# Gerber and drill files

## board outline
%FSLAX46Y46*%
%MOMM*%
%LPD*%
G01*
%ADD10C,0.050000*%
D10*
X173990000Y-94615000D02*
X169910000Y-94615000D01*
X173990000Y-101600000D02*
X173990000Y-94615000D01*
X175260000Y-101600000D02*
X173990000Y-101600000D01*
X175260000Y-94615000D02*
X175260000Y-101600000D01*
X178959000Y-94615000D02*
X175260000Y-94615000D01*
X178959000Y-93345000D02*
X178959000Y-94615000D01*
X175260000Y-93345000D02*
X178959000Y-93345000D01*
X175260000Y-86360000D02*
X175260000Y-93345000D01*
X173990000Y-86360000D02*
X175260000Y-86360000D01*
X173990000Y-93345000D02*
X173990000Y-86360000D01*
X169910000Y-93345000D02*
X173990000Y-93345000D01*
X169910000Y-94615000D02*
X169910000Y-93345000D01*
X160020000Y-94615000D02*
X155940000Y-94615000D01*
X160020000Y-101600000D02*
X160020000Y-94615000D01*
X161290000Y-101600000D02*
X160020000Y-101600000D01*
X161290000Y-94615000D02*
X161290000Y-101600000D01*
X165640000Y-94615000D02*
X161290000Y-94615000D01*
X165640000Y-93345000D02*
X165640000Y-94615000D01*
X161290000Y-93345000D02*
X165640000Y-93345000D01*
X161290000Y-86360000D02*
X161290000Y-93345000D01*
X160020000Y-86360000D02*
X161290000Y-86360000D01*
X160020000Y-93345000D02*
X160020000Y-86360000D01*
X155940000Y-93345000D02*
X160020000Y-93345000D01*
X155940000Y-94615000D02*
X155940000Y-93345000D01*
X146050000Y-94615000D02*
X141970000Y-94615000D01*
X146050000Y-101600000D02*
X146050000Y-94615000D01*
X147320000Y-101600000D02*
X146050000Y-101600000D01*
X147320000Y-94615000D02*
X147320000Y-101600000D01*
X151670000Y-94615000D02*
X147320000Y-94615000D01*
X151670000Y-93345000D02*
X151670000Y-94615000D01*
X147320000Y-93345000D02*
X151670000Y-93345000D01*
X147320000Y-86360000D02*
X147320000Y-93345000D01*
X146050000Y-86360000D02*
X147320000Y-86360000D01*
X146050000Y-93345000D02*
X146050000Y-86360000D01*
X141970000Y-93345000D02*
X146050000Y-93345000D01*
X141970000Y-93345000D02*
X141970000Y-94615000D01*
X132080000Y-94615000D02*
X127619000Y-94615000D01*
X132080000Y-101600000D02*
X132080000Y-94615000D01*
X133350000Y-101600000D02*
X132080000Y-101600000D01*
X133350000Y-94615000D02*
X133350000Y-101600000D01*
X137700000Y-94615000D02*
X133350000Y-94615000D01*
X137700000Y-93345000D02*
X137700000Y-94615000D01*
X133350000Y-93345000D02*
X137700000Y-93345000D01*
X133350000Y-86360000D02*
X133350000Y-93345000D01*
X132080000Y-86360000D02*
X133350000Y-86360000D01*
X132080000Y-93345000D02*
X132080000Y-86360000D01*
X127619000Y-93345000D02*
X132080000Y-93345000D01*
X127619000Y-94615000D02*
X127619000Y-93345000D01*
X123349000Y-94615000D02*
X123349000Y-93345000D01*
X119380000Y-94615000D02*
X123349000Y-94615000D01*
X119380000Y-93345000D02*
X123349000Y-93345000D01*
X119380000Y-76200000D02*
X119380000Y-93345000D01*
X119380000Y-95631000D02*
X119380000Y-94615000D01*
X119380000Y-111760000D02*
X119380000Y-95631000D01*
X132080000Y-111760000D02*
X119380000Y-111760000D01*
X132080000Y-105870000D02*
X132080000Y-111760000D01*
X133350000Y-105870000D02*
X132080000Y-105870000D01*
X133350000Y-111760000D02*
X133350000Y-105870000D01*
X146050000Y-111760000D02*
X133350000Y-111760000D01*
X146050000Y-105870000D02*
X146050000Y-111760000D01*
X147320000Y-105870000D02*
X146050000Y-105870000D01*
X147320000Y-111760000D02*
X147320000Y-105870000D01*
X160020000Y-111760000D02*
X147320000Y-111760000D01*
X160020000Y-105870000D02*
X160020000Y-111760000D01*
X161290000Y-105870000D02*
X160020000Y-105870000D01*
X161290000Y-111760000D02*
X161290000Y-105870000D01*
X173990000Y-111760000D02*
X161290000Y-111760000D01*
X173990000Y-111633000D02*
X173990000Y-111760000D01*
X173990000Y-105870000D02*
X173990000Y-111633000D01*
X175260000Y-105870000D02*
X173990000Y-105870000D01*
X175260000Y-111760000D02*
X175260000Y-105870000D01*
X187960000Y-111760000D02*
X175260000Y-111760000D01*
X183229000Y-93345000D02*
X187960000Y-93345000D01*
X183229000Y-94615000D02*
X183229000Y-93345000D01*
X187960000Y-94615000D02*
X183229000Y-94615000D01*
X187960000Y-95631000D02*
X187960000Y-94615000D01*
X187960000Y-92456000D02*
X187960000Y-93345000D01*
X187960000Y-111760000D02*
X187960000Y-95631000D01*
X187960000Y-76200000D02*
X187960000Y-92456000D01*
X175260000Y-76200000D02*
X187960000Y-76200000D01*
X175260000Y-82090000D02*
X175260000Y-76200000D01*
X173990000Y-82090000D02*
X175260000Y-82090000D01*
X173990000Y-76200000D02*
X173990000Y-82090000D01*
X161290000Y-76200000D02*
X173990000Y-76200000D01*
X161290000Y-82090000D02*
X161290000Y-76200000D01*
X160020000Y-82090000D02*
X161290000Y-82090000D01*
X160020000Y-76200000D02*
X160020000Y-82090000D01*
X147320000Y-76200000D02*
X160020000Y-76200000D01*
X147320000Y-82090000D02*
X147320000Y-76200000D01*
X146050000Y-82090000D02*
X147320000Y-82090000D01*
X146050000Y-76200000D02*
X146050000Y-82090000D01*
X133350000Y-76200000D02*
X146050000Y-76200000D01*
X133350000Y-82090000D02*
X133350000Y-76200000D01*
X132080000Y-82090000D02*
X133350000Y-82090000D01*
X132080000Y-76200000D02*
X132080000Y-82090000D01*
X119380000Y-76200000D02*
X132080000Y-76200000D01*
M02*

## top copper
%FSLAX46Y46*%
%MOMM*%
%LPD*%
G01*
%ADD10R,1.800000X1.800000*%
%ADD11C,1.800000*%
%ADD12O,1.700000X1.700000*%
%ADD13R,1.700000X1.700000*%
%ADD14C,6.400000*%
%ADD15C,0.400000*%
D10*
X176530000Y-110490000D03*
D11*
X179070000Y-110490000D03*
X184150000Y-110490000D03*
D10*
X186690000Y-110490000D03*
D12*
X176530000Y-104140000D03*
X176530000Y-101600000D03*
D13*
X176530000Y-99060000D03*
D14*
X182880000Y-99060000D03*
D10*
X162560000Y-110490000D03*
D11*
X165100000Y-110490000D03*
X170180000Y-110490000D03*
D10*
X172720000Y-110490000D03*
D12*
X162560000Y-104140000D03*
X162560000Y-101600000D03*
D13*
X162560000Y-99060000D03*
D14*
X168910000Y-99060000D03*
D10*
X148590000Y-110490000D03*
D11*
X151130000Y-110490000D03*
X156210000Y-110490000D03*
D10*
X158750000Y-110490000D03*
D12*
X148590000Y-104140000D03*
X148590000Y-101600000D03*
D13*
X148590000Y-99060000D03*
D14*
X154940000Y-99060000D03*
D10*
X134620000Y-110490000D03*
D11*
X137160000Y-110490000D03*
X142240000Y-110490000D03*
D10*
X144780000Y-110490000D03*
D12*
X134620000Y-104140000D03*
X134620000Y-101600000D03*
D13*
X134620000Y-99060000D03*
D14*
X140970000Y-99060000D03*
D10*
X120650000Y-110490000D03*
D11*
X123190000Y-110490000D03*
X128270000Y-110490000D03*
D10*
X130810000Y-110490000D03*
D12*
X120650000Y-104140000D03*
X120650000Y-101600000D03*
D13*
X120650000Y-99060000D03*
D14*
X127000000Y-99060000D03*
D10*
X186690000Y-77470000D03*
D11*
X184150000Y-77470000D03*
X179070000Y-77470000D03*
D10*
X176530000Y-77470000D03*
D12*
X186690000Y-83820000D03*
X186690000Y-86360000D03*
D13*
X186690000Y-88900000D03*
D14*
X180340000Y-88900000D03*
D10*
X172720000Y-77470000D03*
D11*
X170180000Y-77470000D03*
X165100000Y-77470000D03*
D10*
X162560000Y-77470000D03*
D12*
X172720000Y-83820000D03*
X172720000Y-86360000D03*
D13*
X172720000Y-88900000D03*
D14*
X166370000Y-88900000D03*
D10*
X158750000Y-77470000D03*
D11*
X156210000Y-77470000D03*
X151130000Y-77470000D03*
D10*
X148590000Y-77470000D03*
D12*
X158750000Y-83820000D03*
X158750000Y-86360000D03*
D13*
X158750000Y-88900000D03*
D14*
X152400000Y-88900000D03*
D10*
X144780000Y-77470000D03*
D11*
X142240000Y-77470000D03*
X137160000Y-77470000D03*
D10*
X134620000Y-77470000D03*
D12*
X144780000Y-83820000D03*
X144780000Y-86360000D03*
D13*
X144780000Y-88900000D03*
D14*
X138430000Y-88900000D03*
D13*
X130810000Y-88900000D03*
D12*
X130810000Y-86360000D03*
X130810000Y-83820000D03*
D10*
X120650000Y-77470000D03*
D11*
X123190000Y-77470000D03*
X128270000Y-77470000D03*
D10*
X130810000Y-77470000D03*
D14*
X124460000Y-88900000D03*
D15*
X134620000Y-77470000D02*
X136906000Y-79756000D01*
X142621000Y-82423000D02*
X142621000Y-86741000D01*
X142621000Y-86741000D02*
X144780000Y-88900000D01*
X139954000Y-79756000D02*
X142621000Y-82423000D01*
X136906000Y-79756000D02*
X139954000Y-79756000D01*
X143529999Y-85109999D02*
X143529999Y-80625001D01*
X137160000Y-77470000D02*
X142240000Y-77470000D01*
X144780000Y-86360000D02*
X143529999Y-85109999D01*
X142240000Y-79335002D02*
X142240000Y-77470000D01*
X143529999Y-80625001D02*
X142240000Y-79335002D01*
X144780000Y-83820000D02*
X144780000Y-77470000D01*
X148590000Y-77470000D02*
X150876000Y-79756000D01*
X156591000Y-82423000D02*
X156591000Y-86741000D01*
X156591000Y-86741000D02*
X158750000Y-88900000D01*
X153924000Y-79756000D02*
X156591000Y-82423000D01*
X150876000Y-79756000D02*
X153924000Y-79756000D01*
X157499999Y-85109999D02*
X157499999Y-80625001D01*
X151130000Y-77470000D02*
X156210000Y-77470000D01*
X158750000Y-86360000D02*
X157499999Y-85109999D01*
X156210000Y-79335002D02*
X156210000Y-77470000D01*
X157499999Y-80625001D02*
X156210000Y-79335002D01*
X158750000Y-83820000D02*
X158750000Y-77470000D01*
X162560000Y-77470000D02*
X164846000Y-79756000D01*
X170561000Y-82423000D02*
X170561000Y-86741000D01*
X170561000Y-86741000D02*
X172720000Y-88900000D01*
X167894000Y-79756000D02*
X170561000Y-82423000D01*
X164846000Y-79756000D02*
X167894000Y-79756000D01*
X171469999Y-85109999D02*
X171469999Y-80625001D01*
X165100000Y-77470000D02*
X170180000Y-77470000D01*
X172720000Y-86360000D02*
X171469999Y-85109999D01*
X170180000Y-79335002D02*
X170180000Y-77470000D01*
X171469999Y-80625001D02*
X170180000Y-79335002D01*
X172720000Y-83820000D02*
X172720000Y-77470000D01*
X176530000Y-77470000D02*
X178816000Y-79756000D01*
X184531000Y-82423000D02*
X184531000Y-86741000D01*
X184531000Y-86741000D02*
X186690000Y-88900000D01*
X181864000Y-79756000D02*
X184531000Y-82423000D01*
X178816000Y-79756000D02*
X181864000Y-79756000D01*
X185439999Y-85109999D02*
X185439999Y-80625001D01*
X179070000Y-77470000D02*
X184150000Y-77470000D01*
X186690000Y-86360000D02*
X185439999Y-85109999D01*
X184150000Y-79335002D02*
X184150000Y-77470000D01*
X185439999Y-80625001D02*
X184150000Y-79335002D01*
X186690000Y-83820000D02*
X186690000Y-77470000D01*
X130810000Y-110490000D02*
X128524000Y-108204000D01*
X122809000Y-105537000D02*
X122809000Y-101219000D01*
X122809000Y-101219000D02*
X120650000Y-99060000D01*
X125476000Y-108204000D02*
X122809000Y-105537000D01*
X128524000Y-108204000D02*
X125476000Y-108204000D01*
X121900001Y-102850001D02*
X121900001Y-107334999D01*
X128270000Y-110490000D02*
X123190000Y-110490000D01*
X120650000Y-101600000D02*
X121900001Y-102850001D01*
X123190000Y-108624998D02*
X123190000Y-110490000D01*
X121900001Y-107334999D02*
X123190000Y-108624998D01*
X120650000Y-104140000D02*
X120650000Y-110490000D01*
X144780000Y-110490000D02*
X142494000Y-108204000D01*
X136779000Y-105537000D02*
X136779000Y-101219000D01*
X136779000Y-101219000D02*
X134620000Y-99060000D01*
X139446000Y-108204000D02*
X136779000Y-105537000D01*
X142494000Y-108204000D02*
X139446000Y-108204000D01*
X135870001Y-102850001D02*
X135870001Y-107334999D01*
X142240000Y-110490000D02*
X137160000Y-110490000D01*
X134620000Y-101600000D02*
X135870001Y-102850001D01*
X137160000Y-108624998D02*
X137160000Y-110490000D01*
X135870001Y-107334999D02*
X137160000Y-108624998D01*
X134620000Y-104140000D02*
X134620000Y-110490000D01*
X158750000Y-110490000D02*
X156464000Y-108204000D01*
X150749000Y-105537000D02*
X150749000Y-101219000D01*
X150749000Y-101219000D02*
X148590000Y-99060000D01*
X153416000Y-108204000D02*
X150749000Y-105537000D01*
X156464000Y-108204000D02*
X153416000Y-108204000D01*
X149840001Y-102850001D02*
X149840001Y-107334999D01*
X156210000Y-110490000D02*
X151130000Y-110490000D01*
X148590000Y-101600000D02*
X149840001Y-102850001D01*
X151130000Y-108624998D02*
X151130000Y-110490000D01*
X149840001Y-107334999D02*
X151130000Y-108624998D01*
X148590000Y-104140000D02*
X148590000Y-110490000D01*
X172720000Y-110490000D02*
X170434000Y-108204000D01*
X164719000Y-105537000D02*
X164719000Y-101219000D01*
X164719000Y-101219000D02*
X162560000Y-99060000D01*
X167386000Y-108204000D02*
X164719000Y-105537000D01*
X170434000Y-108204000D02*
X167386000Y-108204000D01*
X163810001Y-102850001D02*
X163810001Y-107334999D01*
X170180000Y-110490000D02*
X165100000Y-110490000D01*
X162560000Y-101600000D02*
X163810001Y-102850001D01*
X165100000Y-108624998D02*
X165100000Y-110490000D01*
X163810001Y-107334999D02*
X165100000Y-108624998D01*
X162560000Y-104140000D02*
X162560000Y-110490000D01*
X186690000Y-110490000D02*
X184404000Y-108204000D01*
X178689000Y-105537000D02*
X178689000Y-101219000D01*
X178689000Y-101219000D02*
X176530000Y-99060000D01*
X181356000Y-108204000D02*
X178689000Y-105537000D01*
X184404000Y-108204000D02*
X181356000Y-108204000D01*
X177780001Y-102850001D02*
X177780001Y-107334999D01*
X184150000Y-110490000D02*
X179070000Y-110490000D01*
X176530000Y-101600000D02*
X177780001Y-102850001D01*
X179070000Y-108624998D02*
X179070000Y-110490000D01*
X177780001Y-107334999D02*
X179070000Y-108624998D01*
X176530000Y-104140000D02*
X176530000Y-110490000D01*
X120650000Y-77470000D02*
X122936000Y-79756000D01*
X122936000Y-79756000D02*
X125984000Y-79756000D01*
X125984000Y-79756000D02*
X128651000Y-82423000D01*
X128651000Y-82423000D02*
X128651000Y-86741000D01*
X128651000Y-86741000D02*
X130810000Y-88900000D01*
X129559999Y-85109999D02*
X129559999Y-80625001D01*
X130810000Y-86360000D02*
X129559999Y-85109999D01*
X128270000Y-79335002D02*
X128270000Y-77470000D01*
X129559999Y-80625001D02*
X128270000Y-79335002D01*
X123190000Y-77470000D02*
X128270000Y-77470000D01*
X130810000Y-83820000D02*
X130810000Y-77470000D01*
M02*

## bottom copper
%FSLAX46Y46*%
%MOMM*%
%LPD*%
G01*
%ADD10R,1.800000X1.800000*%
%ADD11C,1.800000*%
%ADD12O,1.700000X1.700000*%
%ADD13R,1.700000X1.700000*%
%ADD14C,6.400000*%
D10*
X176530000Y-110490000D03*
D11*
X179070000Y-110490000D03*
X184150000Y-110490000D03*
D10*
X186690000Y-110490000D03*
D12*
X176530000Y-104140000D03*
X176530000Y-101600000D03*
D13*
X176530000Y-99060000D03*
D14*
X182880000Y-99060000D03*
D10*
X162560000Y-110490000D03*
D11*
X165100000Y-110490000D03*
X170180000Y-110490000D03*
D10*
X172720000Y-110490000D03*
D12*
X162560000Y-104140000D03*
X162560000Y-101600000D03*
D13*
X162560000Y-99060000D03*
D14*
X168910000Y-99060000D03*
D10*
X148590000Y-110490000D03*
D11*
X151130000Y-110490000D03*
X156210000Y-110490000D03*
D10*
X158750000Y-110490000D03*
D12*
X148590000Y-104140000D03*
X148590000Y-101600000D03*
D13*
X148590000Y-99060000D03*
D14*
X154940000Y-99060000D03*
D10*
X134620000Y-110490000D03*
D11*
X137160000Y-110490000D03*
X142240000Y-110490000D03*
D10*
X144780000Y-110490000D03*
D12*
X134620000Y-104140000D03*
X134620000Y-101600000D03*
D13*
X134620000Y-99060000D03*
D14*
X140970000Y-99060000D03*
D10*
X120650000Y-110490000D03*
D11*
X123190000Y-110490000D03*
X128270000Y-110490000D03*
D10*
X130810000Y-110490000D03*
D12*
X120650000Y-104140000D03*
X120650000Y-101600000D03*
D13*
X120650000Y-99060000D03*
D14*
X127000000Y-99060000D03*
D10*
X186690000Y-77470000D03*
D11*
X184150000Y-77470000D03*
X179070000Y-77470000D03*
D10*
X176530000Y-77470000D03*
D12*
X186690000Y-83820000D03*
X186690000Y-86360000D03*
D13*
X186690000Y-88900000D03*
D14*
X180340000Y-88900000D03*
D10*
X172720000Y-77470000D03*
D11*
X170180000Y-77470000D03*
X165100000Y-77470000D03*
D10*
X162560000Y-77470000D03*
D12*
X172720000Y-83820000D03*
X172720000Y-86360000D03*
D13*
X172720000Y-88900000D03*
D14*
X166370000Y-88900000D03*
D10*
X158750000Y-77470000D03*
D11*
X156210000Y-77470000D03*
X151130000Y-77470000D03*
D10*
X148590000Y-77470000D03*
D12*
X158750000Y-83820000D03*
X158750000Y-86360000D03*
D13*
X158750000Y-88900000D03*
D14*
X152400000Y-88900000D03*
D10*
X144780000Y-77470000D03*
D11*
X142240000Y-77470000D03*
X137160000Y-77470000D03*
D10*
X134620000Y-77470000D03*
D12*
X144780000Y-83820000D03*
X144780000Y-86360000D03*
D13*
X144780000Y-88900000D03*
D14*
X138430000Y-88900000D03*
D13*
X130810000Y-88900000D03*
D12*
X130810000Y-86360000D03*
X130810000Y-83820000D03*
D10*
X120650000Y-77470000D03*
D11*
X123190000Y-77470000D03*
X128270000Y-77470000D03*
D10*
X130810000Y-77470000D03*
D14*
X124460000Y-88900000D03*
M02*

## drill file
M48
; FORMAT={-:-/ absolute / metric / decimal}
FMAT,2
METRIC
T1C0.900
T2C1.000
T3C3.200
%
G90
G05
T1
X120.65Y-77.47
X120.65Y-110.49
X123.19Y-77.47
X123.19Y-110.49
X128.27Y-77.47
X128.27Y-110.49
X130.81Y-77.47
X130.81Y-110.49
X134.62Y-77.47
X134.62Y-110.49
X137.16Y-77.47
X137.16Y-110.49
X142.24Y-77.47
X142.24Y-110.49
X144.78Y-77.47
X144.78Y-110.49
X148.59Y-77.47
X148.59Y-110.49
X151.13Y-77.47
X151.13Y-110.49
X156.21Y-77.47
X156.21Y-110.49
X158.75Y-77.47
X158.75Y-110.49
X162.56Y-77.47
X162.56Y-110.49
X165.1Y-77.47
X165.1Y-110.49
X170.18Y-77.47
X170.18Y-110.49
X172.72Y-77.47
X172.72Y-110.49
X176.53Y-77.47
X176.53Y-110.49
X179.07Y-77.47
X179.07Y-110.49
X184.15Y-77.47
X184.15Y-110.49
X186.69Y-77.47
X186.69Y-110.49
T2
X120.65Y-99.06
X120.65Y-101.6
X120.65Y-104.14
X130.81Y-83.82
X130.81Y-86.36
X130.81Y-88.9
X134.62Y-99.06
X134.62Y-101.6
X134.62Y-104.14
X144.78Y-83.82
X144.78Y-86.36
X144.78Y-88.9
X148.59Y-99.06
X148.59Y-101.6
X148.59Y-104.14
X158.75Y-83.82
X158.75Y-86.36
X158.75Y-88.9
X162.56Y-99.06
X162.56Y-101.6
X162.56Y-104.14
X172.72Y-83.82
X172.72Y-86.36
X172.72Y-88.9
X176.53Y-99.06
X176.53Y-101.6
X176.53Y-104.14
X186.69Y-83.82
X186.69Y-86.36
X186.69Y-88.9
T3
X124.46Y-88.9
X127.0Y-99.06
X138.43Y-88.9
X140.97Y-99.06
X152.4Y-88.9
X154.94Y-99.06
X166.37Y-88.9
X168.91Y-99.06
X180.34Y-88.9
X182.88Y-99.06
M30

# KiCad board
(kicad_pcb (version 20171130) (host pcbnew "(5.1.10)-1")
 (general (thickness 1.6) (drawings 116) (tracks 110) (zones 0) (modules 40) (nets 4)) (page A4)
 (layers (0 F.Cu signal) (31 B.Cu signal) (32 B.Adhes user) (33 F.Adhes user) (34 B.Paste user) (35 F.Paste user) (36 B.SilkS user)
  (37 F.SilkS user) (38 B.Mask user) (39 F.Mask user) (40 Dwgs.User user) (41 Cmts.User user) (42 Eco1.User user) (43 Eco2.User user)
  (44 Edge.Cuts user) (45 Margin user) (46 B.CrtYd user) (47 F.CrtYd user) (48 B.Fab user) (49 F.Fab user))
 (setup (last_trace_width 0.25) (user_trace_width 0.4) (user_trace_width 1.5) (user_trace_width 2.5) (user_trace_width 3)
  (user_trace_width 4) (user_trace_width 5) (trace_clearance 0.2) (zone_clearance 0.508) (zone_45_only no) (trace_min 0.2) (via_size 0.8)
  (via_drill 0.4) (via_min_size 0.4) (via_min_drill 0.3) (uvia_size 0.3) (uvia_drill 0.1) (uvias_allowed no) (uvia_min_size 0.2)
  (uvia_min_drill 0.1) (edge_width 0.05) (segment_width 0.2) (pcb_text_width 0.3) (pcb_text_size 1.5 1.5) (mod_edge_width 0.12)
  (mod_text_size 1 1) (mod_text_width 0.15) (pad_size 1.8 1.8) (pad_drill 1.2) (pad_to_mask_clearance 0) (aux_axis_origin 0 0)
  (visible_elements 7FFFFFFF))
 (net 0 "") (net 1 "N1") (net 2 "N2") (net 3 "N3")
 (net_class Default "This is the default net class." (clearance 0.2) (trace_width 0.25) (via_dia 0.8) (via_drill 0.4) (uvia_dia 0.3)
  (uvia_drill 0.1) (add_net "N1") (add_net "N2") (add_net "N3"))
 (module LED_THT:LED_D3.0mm (layer F.Cu) (at 176.53 110.49)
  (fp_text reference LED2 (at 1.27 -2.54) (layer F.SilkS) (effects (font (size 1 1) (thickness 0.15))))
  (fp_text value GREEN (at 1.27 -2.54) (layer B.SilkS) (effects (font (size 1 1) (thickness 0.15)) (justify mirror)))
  (pad 1 thru_hole rect (at 0 0) (size 1.8 1.8) (drill 0.9) (layers *.Cu *.Mask))
  (pad 2 thru_hole circle (at 2.54 0) (size 1.8 1.8) (drill 0.9) (layers *.Cu *.Mask)))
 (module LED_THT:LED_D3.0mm (layer F.Cu) (at 186.69 110.49 180)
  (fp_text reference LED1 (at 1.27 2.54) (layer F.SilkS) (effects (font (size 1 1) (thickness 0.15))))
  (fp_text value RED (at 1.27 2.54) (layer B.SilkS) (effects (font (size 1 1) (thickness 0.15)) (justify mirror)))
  (pad 2 thru_hole circle (at 2.54 0 180) (size 1.8 1.8) (drill 0.9) (layers *.Cu *.Mask))
  (pad 1 thru_hole rect (at 0 0 180) (size 1.8 1.8) (drill 0.9) (layers *.Cu *.Mask)))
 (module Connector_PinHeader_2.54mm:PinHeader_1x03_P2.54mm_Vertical (layer F.Cu) (at 176.53 99.06)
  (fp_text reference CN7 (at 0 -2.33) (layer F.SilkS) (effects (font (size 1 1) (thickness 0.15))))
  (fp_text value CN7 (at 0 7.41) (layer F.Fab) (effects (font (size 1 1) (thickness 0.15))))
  (pad 3 thru_hole oval (at 0 5.08) (size 1.7 1.7) (drill 1) (layers *.Cu *.Mask))
  (pad 2 thru_hole oval (at 0 2.54) (size 1.7 1.7) (drill 1) (layers *.Cu *.Mask))
  (pad 1 thru_hole rect (at 0 0) (size 1.7 1.7) (drill 1) (layers *.Cu *.Mask)))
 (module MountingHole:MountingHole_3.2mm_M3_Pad (layer F.Cu) (at 182.88 99.06 180)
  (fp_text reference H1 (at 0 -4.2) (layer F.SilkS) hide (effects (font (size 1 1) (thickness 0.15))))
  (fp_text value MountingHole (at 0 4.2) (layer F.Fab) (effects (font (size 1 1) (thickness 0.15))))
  (pad 1 thru_hole circle (at 0 0 180) (size 6.4 6.4) (drill 3.2) (layers *.Cu *.Mask)))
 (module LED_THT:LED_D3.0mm (layer F.Cu) (at 162.56 110.49)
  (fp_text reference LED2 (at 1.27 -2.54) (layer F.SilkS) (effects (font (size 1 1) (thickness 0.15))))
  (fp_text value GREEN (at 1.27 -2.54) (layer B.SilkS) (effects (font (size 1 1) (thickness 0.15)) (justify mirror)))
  (pad 1 thru_hole rect (at 0 0) (size 1.8 1.8) (drill 0.9) (layers *.Cu *.Mask))
  (pad 2 thru_hole circle (at 2.54 0) (size 1.8 1.8) (drill 0.9) (layers *.Cu *.Mask)))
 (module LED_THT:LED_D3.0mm (layer F.Cu) (at 172.72 110.49 180)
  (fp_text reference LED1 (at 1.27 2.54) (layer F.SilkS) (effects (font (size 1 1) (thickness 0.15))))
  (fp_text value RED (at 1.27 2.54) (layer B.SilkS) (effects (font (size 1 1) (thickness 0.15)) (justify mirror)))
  (pad 2 thru_hole circle (at 2.54 0 180) (size 1.8 1.8) (drill 0.9) (layers *.Cu *.Mask))
  (pad 1 thru_hole rect (at 0 0 180) (size 1.8 1.8) (drill 0.9) (layers *.Cu *.Mask)))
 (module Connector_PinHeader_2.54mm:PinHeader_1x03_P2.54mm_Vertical (layer F.Cu) (at 162.56 99.06)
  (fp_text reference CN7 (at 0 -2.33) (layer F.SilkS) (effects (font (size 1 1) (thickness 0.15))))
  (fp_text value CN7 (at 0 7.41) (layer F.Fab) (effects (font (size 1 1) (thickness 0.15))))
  (pad 3 thru_hole oval (at 0 5.08) (size 1.7 1.7) (drill 1) (layers *.Cu *.Mask))
  (pad 2 thru_hole oval (at 0 2.54) (size 1.7 1.7) (drill 1) (layers *.Cu *.Mask))
  (pad 1 thru_hole rect (at 0 0) (size 1.7 1.7) (drill 1) (layers *.Cu *.Mask)))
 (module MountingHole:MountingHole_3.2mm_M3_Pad (layer F.Cu) (at 168.91 99.06 180)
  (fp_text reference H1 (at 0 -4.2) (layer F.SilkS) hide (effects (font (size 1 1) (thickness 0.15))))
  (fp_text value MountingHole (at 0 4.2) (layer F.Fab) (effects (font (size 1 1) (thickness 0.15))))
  (pad 1 thru_hole circle (at 0 0 180) (size 6.4 6.4) (drill 3.2) (layers *.Cu *.Mask)))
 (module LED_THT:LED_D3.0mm (layer F.Cu) (at 148.59 110.49)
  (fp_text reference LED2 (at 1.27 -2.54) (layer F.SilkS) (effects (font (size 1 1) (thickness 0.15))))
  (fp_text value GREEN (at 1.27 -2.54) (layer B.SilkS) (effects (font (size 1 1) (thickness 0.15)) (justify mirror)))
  (pad 1 thru_hole rect (at 0 0) (size 1.8 1.8) (drill 0.9) (layers *.Cu *.Mask))
  (pad 2 thru_hole circle (at 2.54 0) (size 1.8 1.8) (drill 0.9) (layers *.Cu *.Mask)))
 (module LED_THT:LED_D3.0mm (layer F.Cu) (at 158.75 110.49 180)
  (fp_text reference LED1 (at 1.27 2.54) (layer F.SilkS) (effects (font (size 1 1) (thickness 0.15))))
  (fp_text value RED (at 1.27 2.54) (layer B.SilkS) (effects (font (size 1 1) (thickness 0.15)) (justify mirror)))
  (pad 2 thru_hole circle (at 2.54 0 180) (size 1.8 1.8) (drill 0.9) (layers *.Cu *.Mask))
  (pad 1 thru_hole rect (at 0 0 180) (size 1.8 1.8) (drill 0.9) (layers *.Cu *.Mask)))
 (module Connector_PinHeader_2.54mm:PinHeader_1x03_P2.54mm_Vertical (layer F.Cu) (at 148.59 99.06)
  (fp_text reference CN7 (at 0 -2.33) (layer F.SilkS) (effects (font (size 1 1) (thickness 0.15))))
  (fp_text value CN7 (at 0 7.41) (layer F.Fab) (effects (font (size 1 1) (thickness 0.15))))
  (pad 3 thru_hole oval (at 0 5.08) (size 1.7 1.7) (drill 1) (layers *.Cu *.Mask))
  (pad 2 thru_hole oval (at 0 2.54) (size 1.7 1.7) (drill 1) (layers *.Cu *.Mask))
  (pad 1 thru_hole rect (at 0 0) (size 1.7 1.7) (drill 1) (layers *.Cu *.Mask)))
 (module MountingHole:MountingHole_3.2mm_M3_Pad (layer F.Cu) (at 154.94 99.06 180)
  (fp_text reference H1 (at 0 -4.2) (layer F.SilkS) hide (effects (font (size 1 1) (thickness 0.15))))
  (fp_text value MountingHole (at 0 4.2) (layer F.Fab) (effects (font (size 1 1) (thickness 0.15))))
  (pad 1 thru_hole circle (at 0 0 180) (size 6.4 6.4) (drill 3.2) (layers *.Cu *.Mask)))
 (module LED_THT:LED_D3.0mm (layer F.Cu) (at 134.62 110.49)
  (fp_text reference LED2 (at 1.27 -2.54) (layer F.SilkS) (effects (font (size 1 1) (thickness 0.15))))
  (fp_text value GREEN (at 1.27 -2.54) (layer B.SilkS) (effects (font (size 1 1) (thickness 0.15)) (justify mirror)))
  (pad 1 thru_hole rect (at 0 0) (size 1.8 1.8) (drill 0.9) (layers *.Cu *.Mask))
  (pad 2 thru_hole circle (at 2.54 0) (size 1.8 1.8) (drill 0.9) (layers *.Cu *.Mask)))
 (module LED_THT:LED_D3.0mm (layer F.Cu) (at 144.78 110.49 180)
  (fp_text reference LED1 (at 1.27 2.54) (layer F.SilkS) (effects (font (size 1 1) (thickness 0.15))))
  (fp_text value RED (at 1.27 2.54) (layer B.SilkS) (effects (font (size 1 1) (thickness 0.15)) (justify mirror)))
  (pad 2 thru_hole circle (at 2.54 0 180) (size 1.8 1.8) (drill 0.9) (layers *.Cu *.Mask))
  (pad 1 thru_hole rect (at 0 0 180) (size 1.8 1.8) (drill 0.9) (layers *.Cu *.Mask)))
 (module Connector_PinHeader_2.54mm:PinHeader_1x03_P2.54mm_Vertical (layer F.Cu) (at 134.62 99.06)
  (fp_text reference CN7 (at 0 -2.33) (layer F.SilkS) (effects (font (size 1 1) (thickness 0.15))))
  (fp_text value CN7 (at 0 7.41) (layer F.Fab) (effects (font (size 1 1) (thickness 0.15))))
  (pad 3 thru_hole oval (at 0 5.08) (size 1.7 1.7) (drill 1) (layers *.Cu *.Mask))
  (pad 2 thru_hole oval (at 0 2.54) (size 1.7 1.7) (drill 1) (layers *.Cu *.Mask))
  (pad 1 thru_hole rect (at 0 0) (size 1.7 1.7) (drill 1) (layers *.Cu *.Mask)))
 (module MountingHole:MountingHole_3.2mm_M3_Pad (layer F.Cu) (at 140.97 99.06 180)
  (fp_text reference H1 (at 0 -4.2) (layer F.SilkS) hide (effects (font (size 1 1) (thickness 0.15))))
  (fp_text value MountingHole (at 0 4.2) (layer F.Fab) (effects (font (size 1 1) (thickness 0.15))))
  (pad 1 thru_hole circle (at 0 0 180) (size 6.4 6.4) (drill 3.2) (layers *.Cu *.Mask)))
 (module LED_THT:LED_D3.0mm (layer F.Cu) (at 120.65 110.49)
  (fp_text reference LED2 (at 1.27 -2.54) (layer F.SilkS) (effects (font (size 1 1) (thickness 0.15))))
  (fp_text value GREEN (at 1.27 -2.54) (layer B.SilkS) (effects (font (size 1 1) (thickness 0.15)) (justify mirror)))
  (pad 1 thru_hole rect (at 0 0) (size 1.8 1.8) (drill 0.9) (layers *.Cu *.Mask))
  (pad 2 thru_hole circle (at 2.54 0) (size 1.8 1.8) (drill 0.9) (layers *.Cu *.Mask)))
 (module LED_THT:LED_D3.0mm (layer F.Cu) (at 130.81 110.49 180)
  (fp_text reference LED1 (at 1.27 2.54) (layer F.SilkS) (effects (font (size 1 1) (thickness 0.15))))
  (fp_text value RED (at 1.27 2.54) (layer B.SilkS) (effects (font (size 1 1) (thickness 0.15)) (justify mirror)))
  (pad 2 thru_hole circle (at 2.54 0 180) (size 1.8 1.8) (drill 0.9) (layers *.Cu *.Mask))
  (pad 1 thru_hole rect (at 0 0 180) (size 1.8 1.8) (drill 0.9) (layers *.Cu *.Mask)))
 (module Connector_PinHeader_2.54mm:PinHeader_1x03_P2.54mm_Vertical (layer F.Cu) (at 120.65 99.06)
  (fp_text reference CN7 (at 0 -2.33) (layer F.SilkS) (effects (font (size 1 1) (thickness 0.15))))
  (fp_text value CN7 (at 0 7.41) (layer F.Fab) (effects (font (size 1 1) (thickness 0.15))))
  (pad 3 thru_hole oval (at 0 5.08) (size 1.7 1.7) (drill 1) (layers *.Cu *.Mask))
  (pad 2 thru_hole oval (at 0 2.54) (size 1.7 1.7) (drill 1) (layers *.Cu *.Mask))
  (pad 1 thru_hole rect (at 0 0) (size 1.7 1.7) (drill 1) (layers *.Cu *.Mask)))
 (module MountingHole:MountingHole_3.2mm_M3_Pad (layer F.Cu) (at 127 99.06 180)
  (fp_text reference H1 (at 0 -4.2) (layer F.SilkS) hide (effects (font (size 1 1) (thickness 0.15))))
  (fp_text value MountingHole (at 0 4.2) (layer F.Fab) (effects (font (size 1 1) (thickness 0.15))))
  (pad 1 thru_hole circle (at 0 0 180) (size 6.4 6.4) (drill 3.2) (layers *.Cu *.Mask)))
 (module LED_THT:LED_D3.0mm (layer F.Cu) (at 186.69 77.47 180)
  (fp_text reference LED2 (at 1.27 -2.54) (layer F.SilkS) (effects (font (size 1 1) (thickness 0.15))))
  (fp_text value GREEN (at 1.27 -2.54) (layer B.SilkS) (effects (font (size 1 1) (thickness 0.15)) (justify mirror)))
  (pad 1 thru_hole rect (at 0 0 180) (size 1.8 1.8) (drill 0.9) (layers *.Cu *.Mask))
  (pad 2 thru_hole circle (at 2.54 0 180) (size 1.8 1.8) (drill 0.9) (layers *.Cu *.Mask)))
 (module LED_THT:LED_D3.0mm (layer F.Cu) (at 176.53 77.47)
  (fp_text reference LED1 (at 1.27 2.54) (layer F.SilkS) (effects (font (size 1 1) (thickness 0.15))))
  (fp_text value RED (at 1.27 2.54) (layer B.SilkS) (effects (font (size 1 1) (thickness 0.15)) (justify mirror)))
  (pad 2 thru_hole circle (at 2.54 0) (size 1.8 1.8) (drill 0.9) (layers *.Cu *.Mask))
  (pad 1 thru_hole rect (at 0 0) (size 1.8 1.8) (drill 0.9) (layers *.Cu *.Mask)))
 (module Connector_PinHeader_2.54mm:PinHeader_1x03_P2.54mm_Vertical (layer F.Cu) (at 186.69 88.9 180)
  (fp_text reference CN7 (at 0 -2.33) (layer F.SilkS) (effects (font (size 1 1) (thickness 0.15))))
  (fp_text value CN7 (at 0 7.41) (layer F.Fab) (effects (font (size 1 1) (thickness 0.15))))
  (pad 3 thru_hole oval (at 0 5.08 180) (size 1.7 1.7) (drill 1) (layers *.Cu *.Mask))
  (pad 2 thru_hole oval (at 0 2.54 180) (size 1.7 1.7) (drill 1) (layers *.Cu *.Mask))
  (pad 1 thru_hole rect (at 0 0 180) (size 1.7 1.7) (drill 1) (layers *.Cu *.Mask)))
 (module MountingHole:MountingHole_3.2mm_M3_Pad (layer F.Cu) (at 180.34 88.9)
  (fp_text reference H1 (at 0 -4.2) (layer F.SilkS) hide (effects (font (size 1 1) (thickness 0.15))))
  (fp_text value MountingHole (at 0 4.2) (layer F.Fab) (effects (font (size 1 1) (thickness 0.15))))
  (pad 1 thru_hole circle (at 0 0) (size 6.4 6.4) (drill 3.2) (layers *.Cu *.Mask)))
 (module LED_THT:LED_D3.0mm (layer F.Cu) (at 172.72 77.47 180)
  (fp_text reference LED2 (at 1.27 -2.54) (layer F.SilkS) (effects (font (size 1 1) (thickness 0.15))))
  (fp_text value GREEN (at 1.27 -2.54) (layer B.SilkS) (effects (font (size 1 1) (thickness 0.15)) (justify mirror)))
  (pad 1 thru_hole rect (at 0 0 180) (size 1.8 1.8) (drill 0.9) (layers *.Cu *.Mask))
  (pad 2 thru_hole circle (at 2.54 0 180) (size 1.8 1.8) (drill 0.9) (layers *.Cu *.Mask)))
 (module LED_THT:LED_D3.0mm (layer F.Cu) (at 162.56 77.47)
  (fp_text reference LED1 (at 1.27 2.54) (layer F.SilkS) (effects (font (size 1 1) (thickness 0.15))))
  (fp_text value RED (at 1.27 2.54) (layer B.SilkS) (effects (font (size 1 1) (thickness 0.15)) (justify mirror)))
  (pad 2 thru_hole circle (at 2.54 0) (size 1.8 1.8) (drill 0.9) (layers *.Cu *.Mask))
  (pad 1 thru_hole rect (at 0 0) (size 1.8 1.8) (drill 0.9) (layers *.Cu *.Mask)))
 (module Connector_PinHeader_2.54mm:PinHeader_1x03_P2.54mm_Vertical (layer F.Cu) (at 172.72 88.9 180)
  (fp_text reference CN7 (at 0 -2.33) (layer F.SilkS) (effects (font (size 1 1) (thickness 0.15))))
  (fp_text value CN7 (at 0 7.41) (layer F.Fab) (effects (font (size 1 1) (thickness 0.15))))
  (pad 3 thru_hole oval (at 0 5.08 180) (size 1.7 1.7) (drill 1) (layers *.Cu *.Mask))
  (pad 2 thru_hole oval (at 0 2.54 180) (size 1.7 1.7) (drill 1) (layers *.Cu *.Mask))
  (pad 1 thru_hole rect (at 0 0 180) (size 1.7 1.7) (drill 1) (layers *.Cu *.Mask)))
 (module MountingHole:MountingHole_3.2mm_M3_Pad (layer F.Cu) (at 166.37 88.9)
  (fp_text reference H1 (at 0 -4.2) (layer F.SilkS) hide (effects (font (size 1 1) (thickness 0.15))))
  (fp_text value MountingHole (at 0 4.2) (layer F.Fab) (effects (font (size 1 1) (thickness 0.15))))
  (pad 1 thru_hole circle (at 0 0) (size 6.4 6.4) (drill 3.2) (layers *.Cu *.Mask)))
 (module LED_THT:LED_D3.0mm (layer F.Cu) (at 158.75 77.47 180)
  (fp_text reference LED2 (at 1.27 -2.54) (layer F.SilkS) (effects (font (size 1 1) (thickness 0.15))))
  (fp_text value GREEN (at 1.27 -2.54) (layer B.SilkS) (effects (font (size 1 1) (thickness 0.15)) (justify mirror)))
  (pad 1 thru_hole rect (at 0 0 180) (size 1.8 1.8) (drill 0.9) (layers *.Cu *.Mask))
  (pad 2 thru_hole circle (at 2.54 0 180) (size 1.8 1.8) (drill 0.9) (layers *.Cu *.Mask)))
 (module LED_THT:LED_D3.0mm (layer F.Cu) (at 148.59 77.47)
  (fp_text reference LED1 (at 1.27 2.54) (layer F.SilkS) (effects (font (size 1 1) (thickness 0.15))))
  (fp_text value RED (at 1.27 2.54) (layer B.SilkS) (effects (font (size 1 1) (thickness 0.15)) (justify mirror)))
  (pad 2 thru_hole circle (at 2.54 0) (size 1.8 1.8) (drill 0.9) (layers *.Cu *.Mask))
  (pad 1 thru_hole rect (at 0 0) (size 1.8 1.8) (drill 0.9) (layers *.Cu *.Mask)))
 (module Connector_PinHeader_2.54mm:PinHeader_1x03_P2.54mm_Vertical (layer F.Cu) (at 158.75 88.9 180)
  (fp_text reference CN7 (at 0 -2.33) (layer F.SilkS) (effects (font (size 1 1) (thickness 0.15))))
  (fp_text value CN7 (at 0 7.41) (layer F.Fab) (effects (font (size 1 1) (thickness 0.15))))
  (pad 3 thru_hole oval (at 0 5.08 180) (size 1.7 1.7) (drill 1) (layers *.Cu *.Mask))
  (pad 2 thru_hole oval (at 0 2.54 180) (size 1.7 1.7) (drill 1) (layers *.Cu *.Mask))
  (pad 1 thru_hole rect (at 0 0 180) (size 1.7 1.7) (drill 1) (layers *.Cu *.Mask)))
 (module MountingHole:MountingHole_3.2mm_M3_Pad (layer F.Cu) (at 152.4 88.9)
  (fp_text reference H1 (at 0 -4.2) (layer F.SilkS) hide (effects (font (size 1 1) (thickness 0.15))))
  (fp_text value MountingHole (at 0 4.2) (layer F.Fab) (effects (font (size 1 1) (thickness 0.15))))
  (pad 1 thru_hole circle (at 0 0) (size 6.4 6.4) (drill 3.2) (layers *.Cu *.Mask)))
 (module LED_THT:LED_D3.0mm (layer F.Cu) (at 144.78 77.47 180)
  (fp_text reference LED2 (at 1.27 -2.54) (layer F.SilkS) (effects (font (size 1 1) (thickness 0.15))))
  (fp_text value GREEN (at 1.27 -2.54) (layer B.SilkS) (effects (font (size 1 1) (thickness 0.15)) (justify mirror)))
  (pad 1 thru_hole rect (at 0 0 180) (size 1.8 1.8) (drill 0.9) (layers *.Cu *.Mask))
  (pad 2 thru_hole circle (at 2.54 0 180) (size 1.8 1.8) (drill 0.9) (layers *.Cu *.Mask)))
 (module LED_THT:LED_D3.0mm (layer F.Cu) (at 134.62 77.47)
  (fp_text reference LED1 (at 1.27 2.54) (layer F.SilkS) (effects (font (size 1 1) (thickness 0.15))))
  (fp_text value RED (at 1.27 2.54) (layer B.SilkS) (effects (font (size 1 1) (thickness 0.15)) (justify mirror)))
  (pad 2 thru_hole circle (at 2.54 0) (size 1.8 1.8) (drill 0.9) (layers *.Cu *.Mask))
  (pad 1 thru_hole rect (at 0 0) (size 1.8 1.8) (drill 0.9) (layers *.Cu *.Mask)))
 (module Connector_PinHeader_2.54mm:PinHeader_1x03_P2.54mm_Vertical (layer F.Cu) (at 144.78 88.9 180)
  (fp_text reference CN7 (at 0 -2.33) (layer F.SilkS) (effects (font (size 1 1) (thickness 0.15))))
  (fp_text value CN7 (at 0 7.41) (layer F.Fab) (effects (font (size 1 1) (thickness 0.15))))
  (pad 3 thru_hole oval (at 0 5.08 180) (size 1.7 1.7) (drill 1) (layers *.Cu *.Mask))
  (pad 2 thru_hole oval (at 0 2.54 180) (size 1.7 1.7) (drill 1) (layers *.Cu *.Mask))
  (pad 1 thru_hole rect (at 0 0 180) (size 1.7 1.7) (drill 1) (layers *.Cu *.Mask)))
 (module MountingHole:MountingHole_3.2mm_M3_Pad (layer F.Cu) (at 138.43 88.9)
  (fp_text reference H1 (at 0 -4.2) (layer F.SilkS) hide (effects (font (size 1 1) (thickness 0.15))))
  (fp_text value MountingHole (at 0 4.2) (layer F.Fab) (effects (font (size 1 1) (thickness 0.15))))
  (pad 1 thru_hole circle (at 0 0) (size 6.4 6.4) (drill 3.2) (layers *.Cu *.Mask)))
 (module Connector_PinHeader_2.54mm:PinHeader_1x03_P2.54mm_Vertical (layer F.Cu) (at 130.81 88.9 180)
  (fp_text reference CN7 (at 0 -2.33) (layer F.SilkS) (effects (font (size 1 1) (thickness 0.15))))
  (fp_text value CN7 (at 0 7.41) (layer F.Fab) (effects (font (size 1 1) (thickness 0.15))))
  (pad 1 thru_hole rect (at 0 0 180) (size 1.7 1.7) (drill 1) (layers *.Cu *.Mask) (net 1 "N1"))
  (pad 2 thru_hole oval (at 0 2.54 180) (size 1.7 1.7) (drill 1) (layers *.Cu *.Mask) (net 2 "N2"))
  (pad 3 thru_hole oval (at 0 5.08 180) (size 1.7 1.7) (drill 1) (layers *.Cu *.Mask) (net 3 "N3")))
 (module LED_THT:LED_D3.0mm (layer F.Cu) (at 120.65 77.47)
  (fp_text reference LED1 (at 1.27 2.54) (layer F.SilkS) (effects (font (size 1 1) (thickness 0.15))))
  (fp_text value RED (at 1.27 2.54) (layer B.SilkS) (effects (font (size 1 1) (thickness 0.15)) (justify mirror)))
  (pad 1 thru_hole rect (at 0 0) (size 1.8 1.8) (drill 0.9) (layers *.Cu *.Mask) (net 1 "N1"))
  (pad 2 thru_hole circle (at 2.54 0) (size 1.8 1.8) (drill 0.9) (layers *.Cu *.Mask) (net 2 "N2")))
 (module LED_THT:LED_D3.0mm (layer F.Cu) (at 130.81 77.47 180)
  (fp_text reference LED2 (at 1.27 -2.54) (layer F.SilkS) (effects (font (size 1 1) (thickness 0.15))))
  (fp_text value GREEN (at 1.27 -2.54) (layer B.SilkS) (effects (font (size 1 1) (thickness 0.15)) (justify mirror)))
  (pad 2 thru_hole circle (at 2.54 0 180) (size 1.8 1.8) (drill 0.9) (layers *.Cu *.Mask) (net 2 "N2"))
  (pad 1 thru_hole rect (at 0 0 180) (size 1.8 1.8) (drill 0.9) (layers *.Cu *.Mask) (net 3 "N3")))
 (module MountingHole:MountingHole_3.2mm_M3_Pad (layer F.Cu) (at 124.46 88.9)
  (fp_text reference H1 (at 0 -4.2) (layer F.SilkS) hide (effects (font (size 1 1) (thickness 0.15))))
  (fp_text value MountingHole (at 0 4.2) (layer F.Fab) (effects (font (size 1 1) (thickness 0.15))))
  (pad 1 thru_hole circle (at 0 0) (size 6.4 6.4) (drill 3.2) (layers *.Cu *.Mask)))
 (gr_line (start 173.99 94.615) (end 169.91 94.615) (layer Edge.Cuts) (width 0.05))
 (gr_line (start 173.99 101.6) (end 173.99 94.615) (layer Edge.Cuts) (width 0.05))
 (gr_line (start 175.26 101.6) (end 173.99 101.6) (layer Edge.Cuts) (width 0.05))
 (gr_line (start 175.26 94.615) (end 175.26 101.6) (layer Edge.Cuts) (width 0.05))
 (gr_line (start 178.959 94.615) (end 175.26 94.615) (layer Edge.Cuts) (width 0.05))
 (gr_line (start 178.959 93.345) (end 178.959 94.615) (layer Edge.Cuts) (width 0.05))
 (gr_line (start 175.26 93.345) (end 178.959 93.345) (layer Edge.Cuts) (width 0.05))
 (gr_line (start 175.26 86.36) (end 175.26 93.345) (layer Edge.Cuts) (width 0.05))
 (gr_line (start 173.99 86.36) (end 175.26 86.36) (layer Edge.Cuts) (width 0.05))
 (gr_line (start 173.99 93.345) (end 173.99 86.36) (layer Edge.Cuts) (width 0.05))
 (gr_line (start 169.91 93.345) (end 173.99 93.345) (layer Edge.Cuts) (width 0.05))
 (gr_line (start 169.91 94.615) (end 169.91 93.345) (layer Edge.Cuts) (width 0.05))
 (gr_line (start 160.02 94.615) (end 155.94 94.615) (layer Edge.Cuts) (width 0.05))
 (gr_line (start 160.02 101.6) (end 160.02 94.615) (layer Edge.Cuts) (width 0.05))
 (gr_line (start 161.29 101.6) (end 160.02 101.6) (layer Edge.Cuts) (width 0.05))
 (gr_line (start 161.29 94.615) (end 161.29 101.6) (layer Edge.Cuts) (width 0.05))
 (gr_line (start 165.64 94.615) (end 161.29 94.615) (layer Edge.Cuts) (width 0.05))
 (gr_line (start 165.64 93.345) (end 165.64 94.615) (layer Edge.Cuts) (width 0.05))
 (gr_line (start 161.29 93.345) (end 165.64 93.345) (layer Edge.Cuts) (width 0.05))
 (gr_line (start 161.29 86.36) (end 161.29 93.345) (layer Edge.Cuts) (width 0.05))
 (gr_line (start 160.02 86.36) (end 161.29 86.36) (layer Edge.Cuts) (width 0.05))
 (gr_line (start 160.02 93.345) (end 160.02 86.36) (layer Edge.Cuts) (width 0.05))
 (gr_line (start 155.94 93.345) (end 160.02 93.345) (layer Edge.Cuts) (width 0.05))
 (gr_line (start 155.94 94.615) (end 155.94 93.345) (layer Edge.Cuts) (width 0.05))
 (gr_line (start 146.05 94.615) (end 141.97 94.615) (layer Edge.Cuts) (width 0.05))
 (gr_line (start 146.05 101.6) (end 146.05 94.615) (layer Edge.Cuts) (width 0.05))
 (gr_line (start 147.32 101.6) (end 146.05 101.6) (layer Edge.Cuts) (width 0.05))
 (gr_line (start 147.32 94.615) (end 147.32 101.6) (layer Edge.Cuts) (width 0.05))
 (gr_line (start 151.67 94.615) (end 147.32 94.615) (layer Edge.Cuts) (width 0.05))
 (gr_line (start 151.67 93.345) (end 151.67 94.615) (layer Edge.Cuts) (width 0.05))
 (gr_line (start 147.32 93.345) (end 151.67 93.345) (layer Edge.Cuts) (width 0.05))
 (gr_line (start 147.32 86.36) (end 147.32 93.345) (layer Edge.Cuts) (width 0.05))
 (gr_line (start 146.05 86.36) (end 147.32 86.36) (layer Edge.Cuts) (width 0.05))
 (gr_line (start 146.05 93.345) (end 146.05 86.36) (layer Edge.Cuts) (width 0.05))
 (gr_line (start 141.97 93.345) (end 146.05 93.345) (layer Edge.Cuts) (width 0.05))
 (gr_line (start 141.97 93.345) (end 141.97 94.615) (layer Edge.Cuts) (width 0.05))
 (gr_line (start 132.08 94.615) (end 127.619 94.615) (layer Edge.Cuts) (width 0.05))
 (gr_line (start 132.08 101.6) (end 132.08 94.615) (layer Edge.Cuts) (width 0.05))
 (gr_line (start 133.35 101.6) (end 132.08 101.6) (layer Edge.Cuts) (width 0.05))
 (gr_line (start 133.35 94.615) (end 133.35 101.6) (layer Edge.Cuts) (width 0.05))
 (gr_line (start 137.7 94.615) (end 133.35 94.615) (layer Edge.Cuts) (width 0.05))
 (gr_line (start 137.7 93.345) (end 137.7 94.615) (layer Edge.Cuts) (width 0.05))
 (gr_line (start 133.35 93.345) (end 137.7 93.345) (layer Edge.Cuts) (width 0.05))
 (gr_line (start 133.35 86.36) (end 133.35 93.345) (layer Edge.Cuts) (width 0.05))
 (gr_line (start 132.08 86.36) (end 133.35 86.36) (layer Edge.Cuts) (width 0.05))
 (gr_line (start 132.08 93.345) (end 132.08 86.36) (layer Edge.Cuts) (width 0.05))
 (gr_line (start 127.619 93.345) (end 132.08 93.345) (layer Edge.Cuts) (width 0.05))
 (gr_line (start 127.619 94.615) (end 127.619 93.345) (layer Edge.Cuts) (width 0.05))
 (gr_line (start 123.349 94.615) (end 123.349 93.345) (layer Edge.Cuts) (width 0.05))
 (gr_line (start 119.38 94.615) (end 123.349 94.615) (layer Edge.Cuts) (width 0.05))
 (gr_line (start 119.38 93.345) (end 123.349 93.345) (layer Edge.Cuts) (width 0.05))
 (gr_line (start 119.38 76.2) (end 119.38 93.345) (layer Edge.Cuts) (width 0.05))
 (gr_line (start 119.38 95.631) (end 119.38 94.615) (layer Edge.Cuts) (width 0.05))
 (gr_line (start 119.38 111.76) (end 119.38 95.631) (layer Edge.Cuts) (width 0.05))
 (gr_line (start 132.08 111.76) (end 119.38 111.76) (layer Edge.Cuts) (width 0.05))
 (gr_line (start 132.08 105.87) (end 132.08 111.76) (layer Edge.Cuts) (width 0.05))
 (gr_line (start 133.35 105.87) (end 132.08 105.87) (layer Edge.Cuts) (width 0.05))
 (gr_line (start 133.35 111.76) (end 133.35 105.87) (layer Edge.Cuts) (width 0.05))
 (gr_line (start 146.05 111.76) (end 133.35 111.76) (layer Edge.Cuts) (width 0.05))
 (gr_line (start 146.05 105.87) (end 146.05 111.76) (layer Edge.Cuts) (width 0.05))
 (gr_line (start 147.32 105.87) (end 146.05 105.87) (layer Edge.Cuts) (width 0.05))
 (gr_line (start 147.32 111.76) (end 147.32 105.87) (layer Edge.Cuts) (width 0.05))
 (gr_line (start 160.02 111.76) (end 147.32 111.76) (layer Edge.Cuts) (width 0.05))
 (gr_line (start 160.02 105.87) (end 160.02 111.76) (layer Edge.Cuts) (width 0.05))
 (gr_line (start 161.29 105.87) (end 160.02 105.87) (layer Edge.Cuts) (width 0.05))
 (gr_line (start 161.29 111.76) (end 161.29 105.87) (layer Edge.Cuts) (width 0.05))
 (gr_line (start 173.99 111.76) (end 161.29 111.76) (layer Edge.Cuts) (width 0.05))
 (gr_line (start 173.99 111.633) (end 173.99 111.76) (layer Edge.Cuts) (width 0.05))
 (gr_line (start 173.99 105.87) (end 173.99 111.633) (layer Edge.Cuts) (width 0.05))
 (gr_line (start 175.26 105.87) (end 173.99 105.87) (layer Edge.Cuts) (width 0.05))
 (gr_line (start 175.26 111.76) (end 175.26 105.87) (layer Edge.Cuts) (width 0.05))
 (gr_line (start 187.96 111.76) (end 175.26 111.76) (layer Edge.Cuts) (width 0.05))
 (gr_line (start 183.229 93.345) (end 187.96 93.345) (layer Edge.Cuts) (width 0.05))
 (gr_line (start 183.229 94.615) (end 183.229 93.345) (layer Edge.Cuts) (width 0.05))
 (gr_line (start 187.96 94.615) (end 183.229 94.615) (layer Edge.Cuts) (width 0.05))
 (gr_line (start 187.96 95.631) (end 187.96 94.615) (layer Edge.Cuts) (width 0.05))
 (gr_line (start 187.96 92.456) (end 187.96 93.345) (layer Edge.Cuts) (width 0.05))
 (gr_line (start 187.96 111.76) (end 187.96 95.631) (layer Edge.Cuts) (width 0.05))
 (gr_line (start 187.96 76.2) (end 187.96 92.456) (layer Edge.Cuts) (width 0.05))
 (gr_line (start 175.26 76.2) (end 187.96 76.2) (layer Edge.Cuts) (width 0.05))
 (gr_line (start 175.26 82.09) (end 175.26 76.2) (layer Edge.Cuts) (width 0.05))
 (gr_line (start 173.99 82.09) (end 175.26 82.09) (layer Edge.Cuts) (width 0.05))
 (gr_line (start 173.99 76.2) (end 173.99 82.09) (layer Edge.Cuts) (width 0.05))
 (gr_line (start 161.29 76.2) (end 173.99 76.2) (layer Edge.Cuts) (width 0.05))
 (gr_line (start 161.29 82.09) (end 161.29 76.2) (layer Edge.Cuts) (width 0.05))
 (gr_line (start 160.02 82.09) (end 161.29 82.09) (layer Edge.Cuts) (width 0.05))
 (gr_line (start 160.02 76.2) (end 160.02 82.09) (layer Edge.Cuts) (width 0.05))
 (gr_line (start 147.32 76.2) (end 160.02 76.2) (layer Edge.Cuts) (width 0.05))
 (gr_line (start 147.32 82.09) (end 147.32 76.2) (layer Edge.Cuts) (width 0.05))
 (gr_line (start 146.05 82.09) (end 147.32 82.09) (layer Edge.Cuts) (width 0.05))
 (gr_line (start 146.05 76.2) (end 146.05 82.09) (layer Edge.Cuts) (width 0.05))
 (gr_line (start 133.35 76.2) (end 146.05 76.2) (layer Edge.Cuts) (width 0.05))
 (gr_line (start 133.35 82.09) (end 133.35 76.2) (layer Edge.Cuts) (width 0.05))
 (gr_line (start 132.08 82.09) (end 133.35 82.09) (layer Edge.Cuts) (width 0.05))
 (gr_line (start 132.08 76.2) (end 132.08 82.09) (layer Edge.Cuts) (width 0.05))
 (gr_line (start 119.38 76.2) (end 132.08 76.2) (layer Edge.Cuts) (width 0.05))
 (segment (start 134.62 77.47) (end 136.906 79.756) (width 0.4) (layer F.Cu) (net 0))
 (segment (start 142.621 82.423) (end 142.621 86.741) (width 0.4) (layer F.Cu) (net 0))
 (segment (start 142.621 86.741) (end 144.78 88.9) (width 0.4) (layer F.Cu) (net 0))
 (segment (start 139.954 79.756) (end 142.621 82.423) (width 0.4) (layer F.Cu) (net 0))
 (segment (start 136.906 79.756) (end 139.954 79.756) (width 0.4) (layer F.Cu) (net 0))
 (segment (start 143.529999 85.109999) (end 143.529999 80.625001) (width 0.4) (layer F.Cu) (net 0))
 (segment (start 137.16 77.47) (end 142.24 77.47) (width 0.4) (layer F.Cu) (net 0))
 (segment (start 144.78 86.36) (end 143.529999 85.109999) (width 0.4) (layer F.Cu) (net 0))
 (segment (start 142.24 79.335002) (end 142.24 77.47) (width 0.4) (layer F.Cu) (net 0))
 (segment (start 143.529999 80.625001) (end 142.24 79.335002) (width 0.4) (layer F.Cu) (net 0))
 (segment (start 144.78 83.82) (end 144.78 77.47) (width 0.4) (layer F.Cu) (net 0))
 (segment (start 148.59 77.47) (end 150.876 79.756) (width 0.4) (layer F.Cu) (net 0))
 (segment (start 156.591 82.423) (end 156.591 86.741) (width 0.4) (layer F.Cu) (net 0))
 (segment (start 156.591 86.741) (end 158.75 88.9) (width 0.4) (layer F.Cu) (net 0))
 (segment (start 153.924 79.756) (end 156.591 82.423) (width 0.4) (layer F.Cu) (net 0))
 (segment (start 150.876 79.756) (end 153.924 79.756) (width 0.4) (layer F.Cu) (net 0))
 (segment (start 157.499999 85.109999) (end 157.499999 80.625001) (width 0.4) (layer F.Cu) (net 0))
 (segment (start 151.13 77.47) (end 156.21 77.47) (width 0.4) (layer F.Cu) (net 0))
 (segment (start 158.75 86.36) (end 157.499999 85.109999) (width 0.4) (layer F.Cu) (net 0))
 (segment (start 156.21 79.335002) (end 156.21 77.47) (width 0.4) (layer F.Cu) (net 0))
 (segment (start 157.499999 80.625001) (end 156.21 79.335002) (width 0.4) (layer F.Cu) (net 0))
 (segment (start 158.75 83.82) (end 158.75 77.47) (width 0.4) (layer F.Cu) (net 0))
 (segment (start 162.56 77.47) (end 164.846 79.756) (width 0.4) (layer F.Cu) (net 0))
 (segment (start 170.561 82.423) (end 170.561 86.741) (width 0.4) (layer F.Cu) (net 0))
 (segment (start 170.561 86.741) (end 172.72 88.9) (width 0.4) (layer F.Cu) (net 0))
 (segment (start 167.894 79.756) (end 170.561 82.423) (width 0.4) (layer F.Cu) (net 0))
 (segment (start 164.846 79.756) (end 167.894 79.756) (width 0.4) (layer F.Cu) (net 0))
 (segment (start 171.469999 85.109999) (end 171.469999 80.625001) (width 0.4) (layer F.Cu) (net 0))
 (segment (start 165.1 77.47) (end 170.18 77.47) (width 0.4) (layer F.Cu) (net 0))
 (segment (start 172.72 86.36) (end 171.469999 85.109999) (width 0.4) (layer F.Cu) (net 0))
 (segment (start 170.18 79.335002) (end 170.18 77.47) (width 0.4) (layer F.Cu) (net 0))
 (segment (start 171.469999 80.625001) (end 170.18 79.335002) (width 0.4) (layer F.Cu) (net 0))
 (segment (start 172.72 83.82) (end 172.72 77.47) (width 0.4) (layer F.Cu) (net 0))
 (segment (start 176.53 77.47) (end 178.816 79.756) (width 0.4) (layer F.Cu) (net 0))
 (segment (start 184.531 82.423) (end 184.531 86.741) (width 0.4) (layer F.Cu) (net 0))
 (segment (start 184.531 86.741) (end 186.69 88.9) (width 0.4) (layer F.Cu) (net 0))
 (segment (start 181.864 79.756) (end 184.531 82.423) (width 0.4) (layer F.Cu) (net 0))
 (segment (start 178.816 79.756) (end 181.864 79.756) (width 0.4) (layer F.Cu) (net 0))
 (segment (start 185.439999 85.109999) (end 185.439999 80.625001) (width 0.4) (layer F.Cu) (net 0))
 (segment (start 179.07 77.47) (end 184.15 77.47) (width 0.4) (layer F.Cu) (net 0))
 (segment (start 186.69 86.36) (end 185.439999 85.109999) (width 0.4) (layer F.Cu) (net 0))
 (segment (start 184.15 79.335002) (end 184.15 77.47) (width 0.4) (layer F.Cu) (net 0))
 (segment (start 185.439999 80.625001) (end 184.15 79.335002) (width 0.4) (layer F.Cu) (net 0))
 (segment (start 186.69 83.82) (end 186.69 77.47) (width 0.4) (layer F.Cu) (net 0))
 (segment (start 130.81 110.49) (end 128.524 108.204) (width 0.4) (layer F.Cu) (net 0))
 (segment (start 122.809 105.537) (end 122.809 101.219) (width 0.4) (layer F.Cu) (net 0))
 (segment (start 122.809 101.219) (end 120.65 99.06) (width 0.4) (layer F.Cu) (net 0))
 (segment (start 125.476 108.204) (end 122.809 105.537) (width 0.4) (layer F.Cu) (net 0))
 (segment (start 128.524 108.204) (end 125.476 108.204) (width 0.4) (layer F.Cu) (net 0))
 (segment (start 121.900001 102.850001) (end 121.900001 107.334999) (width 0.4) (layer F.Cu) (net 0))
 (segment (start 128.27 110.49) (end 123.19 110.49) (width 0.4) (layer F.Cu) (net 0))
 (segment (start 120.65 101.6) (end 121.900001 102.850001) (width 0.4) (layer F.Cu) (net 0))
 (segment (start 123.19 108.624998) (end 123.19 110.49) (width 0.4) (layer F.Cu) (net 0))
 (segment (start 121.900001 107.334999) (end 123.19 108.624998) (width 0.4) (layer F.Cu) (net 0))
 (segment (start 120.65 104.14) (end 120.65 110.49) (width 0.4) (layer F.Cu) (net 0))
 (segment (start 144.78 110.49) (end 142.494 108.204) (width 0.4) (layer F.Cu) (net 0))
 (segment (start 136.779 105.537) (end 136.779 101.219) (width 0.4) (layer F.Cu) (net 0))
 (segment (start 136.779 101.219) (end 134.62 99.06) (width 0.4) (layer F.Cu) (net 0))
 (segment (start 139.446 108.204) (end 136.779 105.537) (width 0.4) (layer F.Cu) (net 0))
 (segment (start 142.494 108.204) (end 139.446 108.204) (width 0.4) (layer F.Cu) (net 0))
 (segment (start 135.870001 102.850001) (end 135.870001 107.334999) (width 0.4) (layer F.Cu) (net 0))
 (segment (start 142.24 110.49) (end 137.16 110.49) (width 0.4) (layer F.Cu) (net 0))
 (segment (start 134.62 101.6) (end 135.870001 102.850001) (width 0.4) (layer F.Cu) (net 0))
 (segment (start 137.16 108.624998) (end 137.16 110.49) (width 0.4) (layer F.Cu) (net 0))
 (segment (start 135.870001 107.334999) (end 137.16 108.624998) (width 0.4) (layer F.Cu) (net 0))
 (segment (start 134.62 104.14) (end 134.62 110.49) (width 0.4) (layer F.Cu) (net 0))
 (segment (start 158.75 110.49) (end 156.464 108.204) (width 0.4) (layer F.Cu) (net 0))
 (segment (start 150.749 105.537) (end 150.749 101.219) (width 0.4) (layer F.Cu) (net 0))
 (segment (start 150.749 101.219) (end 148.59 99.06) (width 0.4) (layer F.Cu) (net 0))
 (segment (start 153.416 108.204) (end 150.749 105.537) (width 0.4) (layer F.Cu) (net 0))
 (segment (start 156.464 108.204) (end 153.416 108.204) (width 0.4) (layer F.Cu) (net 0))
 (segment (start 149.840001 102.850001) (end 149.840001 107.334999) (width 0.4) (layer F.Cu) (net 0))
 (segment (start 156.21 110.49) (end 151.13 110.49) (width 0.4) (layer F.Cu) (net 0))
 (segment (start 148.59 101.6) (end 149.840001 102.850001) (width 0.4) (layer F.Cu) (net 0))
 (segment (start 151.13 108.624998) (end 151.13 110.49) (width 0.4) (layer F.Cu) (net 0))
 (segment (start 149.840001 107.334999) (end 151.13 108.624998) (width 0.4) (layer F.Cu) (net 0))
 (segment (start 148.59 104.14) (end 148.59 110.49) (width 0.4) (layer F.Cu) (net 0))
 (segment (start 172.72 110.49) (end 170.434 108.204) (width 0.4) (layer F.Cu) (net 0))
 (segment (start 164.719 105.537) (end 164.719 101.219) (width 0.4) (layer F.Cu) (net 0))
 (segment (start 164.719 101.219) (end 162.56 99.06) (width 0.4) (layer F.Cu) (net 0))
 (segment (start 167.386 108.204) (end 164.719 105.537) (width 0.4) (layer F.Cu) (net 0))
 (segment (start 170.434 108.204) (end 167.386 108.204) (width 0.4) (layer F.Cu) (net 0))
 (segment (start 163.810001 102.850001) (end 163.810001 107.334999) (width 0.4) (layer F.Cu) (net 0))
 (segment (start 170.18 110.49) (end 165.1 110.49) (width 0.4) (layer F.Cu) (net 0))
 (segment (start 162.56 101.6) (end 163.810001 102.850001) (width 0.4) (layer F.Cu) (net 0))
 (segment (start 165.1 108.624998) (end 165.1 110.49) (width 0.4) (layer F.Cu) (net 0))
 (segment (start 163.810001 107.334999) (end 165.1 108.624998) (width 0.4) (layer F.Cu) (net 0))
 (segment (start 162.56 104.14) (end 162.56 110.49) (width 0.4) (layer F.Cu) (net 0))
 (segment (start 186.69 110.49) (end 184.404 108.204) (width 0.4) (layer F.Cu) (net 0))
 (segment (start 178.689 105.537) (end 178.689 101.219) (width 0.4) (layer F.Cu) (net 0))
 (segment (start 178.689 101.219) (end 176.53 99.06) (width 0.4) (layer F.Cu) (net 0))
 (segment (start 181.356 108.204) (end 178.689 105.537) (width 0.4) (layer F.Cu) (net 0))
 (segment (start 184.404 108.204) (end 181.356 108.204) (width 0.4) (layer F.Cu) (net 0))
 (segment (start 177.780001 102.850001) (end 177.780001 107.334999) (width 0.4) (layer F.Cu) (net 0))
 (segment (start 184.15 110.49) (end 179.07 110.49) (width 0.4) (layer F.Cu) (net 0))
 (segment (start 176.53 101.6) (end 177.780001 102.850001) (width 0.4) (layer F.Cu) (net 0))
 (segment (start 179.07 108.624998) (end 179.07 110.49) (width 0.4) (layer F.Cu) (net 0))
 (segment (start 177.780001 107.334999) (end 179.07 108.624998) (width 0.4) (layer F.Cu) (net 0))
 (segment (start 176.53 104.14) (end 176.53 110.49) (width 0.4) (layer F.Cu) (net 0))
 (segment (start 120.65 77.47) (end 122.936 79.756) (width 0.4) (layer F.Cu) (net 1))
 (segment (start 122.936 79.756) (end 125.984 79.756) (width 0.4) (layer F.Cu) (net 1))
 (segment (start 125.984 79.756) (end 128.651 82.423) (width 0.4) (layer F.Cu) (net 1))
 (segment (start 128.651 82.423) (end 128.651 86.741) (width 0.4) (layer F.Cu) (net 1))
 (segment (start 128.651 86.741) (end 130.81 88.9) (width 0.4) (layer F.Cu) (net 1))
 (segment (start 129.559999 85.109999) (end 129.559999 80.625001) (width 0.4) (layer F.Cu) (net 2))
 (segment (start 130.81 86.36) (end 129.559999 85.109999) (width 0.4) (layer F.Cu) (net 2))
 (segment (start 128.27 79.335002) (end 128.27 77.47) (width 0.4) (layer F.Cu) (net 2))
 (segment (start 129.559999 80.625001) (end 128.27 79.335002) (width 0.4) (layer F.Cu) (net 2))
 (segment (start 123.19 77.47) (end 128.27 77.47) (width 0.4) (layer F.Cu) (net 2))
 (segment (start 130.81 83.82) (end 130.81 77.47) (width 0.4) (layer F.Cu) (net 3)))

